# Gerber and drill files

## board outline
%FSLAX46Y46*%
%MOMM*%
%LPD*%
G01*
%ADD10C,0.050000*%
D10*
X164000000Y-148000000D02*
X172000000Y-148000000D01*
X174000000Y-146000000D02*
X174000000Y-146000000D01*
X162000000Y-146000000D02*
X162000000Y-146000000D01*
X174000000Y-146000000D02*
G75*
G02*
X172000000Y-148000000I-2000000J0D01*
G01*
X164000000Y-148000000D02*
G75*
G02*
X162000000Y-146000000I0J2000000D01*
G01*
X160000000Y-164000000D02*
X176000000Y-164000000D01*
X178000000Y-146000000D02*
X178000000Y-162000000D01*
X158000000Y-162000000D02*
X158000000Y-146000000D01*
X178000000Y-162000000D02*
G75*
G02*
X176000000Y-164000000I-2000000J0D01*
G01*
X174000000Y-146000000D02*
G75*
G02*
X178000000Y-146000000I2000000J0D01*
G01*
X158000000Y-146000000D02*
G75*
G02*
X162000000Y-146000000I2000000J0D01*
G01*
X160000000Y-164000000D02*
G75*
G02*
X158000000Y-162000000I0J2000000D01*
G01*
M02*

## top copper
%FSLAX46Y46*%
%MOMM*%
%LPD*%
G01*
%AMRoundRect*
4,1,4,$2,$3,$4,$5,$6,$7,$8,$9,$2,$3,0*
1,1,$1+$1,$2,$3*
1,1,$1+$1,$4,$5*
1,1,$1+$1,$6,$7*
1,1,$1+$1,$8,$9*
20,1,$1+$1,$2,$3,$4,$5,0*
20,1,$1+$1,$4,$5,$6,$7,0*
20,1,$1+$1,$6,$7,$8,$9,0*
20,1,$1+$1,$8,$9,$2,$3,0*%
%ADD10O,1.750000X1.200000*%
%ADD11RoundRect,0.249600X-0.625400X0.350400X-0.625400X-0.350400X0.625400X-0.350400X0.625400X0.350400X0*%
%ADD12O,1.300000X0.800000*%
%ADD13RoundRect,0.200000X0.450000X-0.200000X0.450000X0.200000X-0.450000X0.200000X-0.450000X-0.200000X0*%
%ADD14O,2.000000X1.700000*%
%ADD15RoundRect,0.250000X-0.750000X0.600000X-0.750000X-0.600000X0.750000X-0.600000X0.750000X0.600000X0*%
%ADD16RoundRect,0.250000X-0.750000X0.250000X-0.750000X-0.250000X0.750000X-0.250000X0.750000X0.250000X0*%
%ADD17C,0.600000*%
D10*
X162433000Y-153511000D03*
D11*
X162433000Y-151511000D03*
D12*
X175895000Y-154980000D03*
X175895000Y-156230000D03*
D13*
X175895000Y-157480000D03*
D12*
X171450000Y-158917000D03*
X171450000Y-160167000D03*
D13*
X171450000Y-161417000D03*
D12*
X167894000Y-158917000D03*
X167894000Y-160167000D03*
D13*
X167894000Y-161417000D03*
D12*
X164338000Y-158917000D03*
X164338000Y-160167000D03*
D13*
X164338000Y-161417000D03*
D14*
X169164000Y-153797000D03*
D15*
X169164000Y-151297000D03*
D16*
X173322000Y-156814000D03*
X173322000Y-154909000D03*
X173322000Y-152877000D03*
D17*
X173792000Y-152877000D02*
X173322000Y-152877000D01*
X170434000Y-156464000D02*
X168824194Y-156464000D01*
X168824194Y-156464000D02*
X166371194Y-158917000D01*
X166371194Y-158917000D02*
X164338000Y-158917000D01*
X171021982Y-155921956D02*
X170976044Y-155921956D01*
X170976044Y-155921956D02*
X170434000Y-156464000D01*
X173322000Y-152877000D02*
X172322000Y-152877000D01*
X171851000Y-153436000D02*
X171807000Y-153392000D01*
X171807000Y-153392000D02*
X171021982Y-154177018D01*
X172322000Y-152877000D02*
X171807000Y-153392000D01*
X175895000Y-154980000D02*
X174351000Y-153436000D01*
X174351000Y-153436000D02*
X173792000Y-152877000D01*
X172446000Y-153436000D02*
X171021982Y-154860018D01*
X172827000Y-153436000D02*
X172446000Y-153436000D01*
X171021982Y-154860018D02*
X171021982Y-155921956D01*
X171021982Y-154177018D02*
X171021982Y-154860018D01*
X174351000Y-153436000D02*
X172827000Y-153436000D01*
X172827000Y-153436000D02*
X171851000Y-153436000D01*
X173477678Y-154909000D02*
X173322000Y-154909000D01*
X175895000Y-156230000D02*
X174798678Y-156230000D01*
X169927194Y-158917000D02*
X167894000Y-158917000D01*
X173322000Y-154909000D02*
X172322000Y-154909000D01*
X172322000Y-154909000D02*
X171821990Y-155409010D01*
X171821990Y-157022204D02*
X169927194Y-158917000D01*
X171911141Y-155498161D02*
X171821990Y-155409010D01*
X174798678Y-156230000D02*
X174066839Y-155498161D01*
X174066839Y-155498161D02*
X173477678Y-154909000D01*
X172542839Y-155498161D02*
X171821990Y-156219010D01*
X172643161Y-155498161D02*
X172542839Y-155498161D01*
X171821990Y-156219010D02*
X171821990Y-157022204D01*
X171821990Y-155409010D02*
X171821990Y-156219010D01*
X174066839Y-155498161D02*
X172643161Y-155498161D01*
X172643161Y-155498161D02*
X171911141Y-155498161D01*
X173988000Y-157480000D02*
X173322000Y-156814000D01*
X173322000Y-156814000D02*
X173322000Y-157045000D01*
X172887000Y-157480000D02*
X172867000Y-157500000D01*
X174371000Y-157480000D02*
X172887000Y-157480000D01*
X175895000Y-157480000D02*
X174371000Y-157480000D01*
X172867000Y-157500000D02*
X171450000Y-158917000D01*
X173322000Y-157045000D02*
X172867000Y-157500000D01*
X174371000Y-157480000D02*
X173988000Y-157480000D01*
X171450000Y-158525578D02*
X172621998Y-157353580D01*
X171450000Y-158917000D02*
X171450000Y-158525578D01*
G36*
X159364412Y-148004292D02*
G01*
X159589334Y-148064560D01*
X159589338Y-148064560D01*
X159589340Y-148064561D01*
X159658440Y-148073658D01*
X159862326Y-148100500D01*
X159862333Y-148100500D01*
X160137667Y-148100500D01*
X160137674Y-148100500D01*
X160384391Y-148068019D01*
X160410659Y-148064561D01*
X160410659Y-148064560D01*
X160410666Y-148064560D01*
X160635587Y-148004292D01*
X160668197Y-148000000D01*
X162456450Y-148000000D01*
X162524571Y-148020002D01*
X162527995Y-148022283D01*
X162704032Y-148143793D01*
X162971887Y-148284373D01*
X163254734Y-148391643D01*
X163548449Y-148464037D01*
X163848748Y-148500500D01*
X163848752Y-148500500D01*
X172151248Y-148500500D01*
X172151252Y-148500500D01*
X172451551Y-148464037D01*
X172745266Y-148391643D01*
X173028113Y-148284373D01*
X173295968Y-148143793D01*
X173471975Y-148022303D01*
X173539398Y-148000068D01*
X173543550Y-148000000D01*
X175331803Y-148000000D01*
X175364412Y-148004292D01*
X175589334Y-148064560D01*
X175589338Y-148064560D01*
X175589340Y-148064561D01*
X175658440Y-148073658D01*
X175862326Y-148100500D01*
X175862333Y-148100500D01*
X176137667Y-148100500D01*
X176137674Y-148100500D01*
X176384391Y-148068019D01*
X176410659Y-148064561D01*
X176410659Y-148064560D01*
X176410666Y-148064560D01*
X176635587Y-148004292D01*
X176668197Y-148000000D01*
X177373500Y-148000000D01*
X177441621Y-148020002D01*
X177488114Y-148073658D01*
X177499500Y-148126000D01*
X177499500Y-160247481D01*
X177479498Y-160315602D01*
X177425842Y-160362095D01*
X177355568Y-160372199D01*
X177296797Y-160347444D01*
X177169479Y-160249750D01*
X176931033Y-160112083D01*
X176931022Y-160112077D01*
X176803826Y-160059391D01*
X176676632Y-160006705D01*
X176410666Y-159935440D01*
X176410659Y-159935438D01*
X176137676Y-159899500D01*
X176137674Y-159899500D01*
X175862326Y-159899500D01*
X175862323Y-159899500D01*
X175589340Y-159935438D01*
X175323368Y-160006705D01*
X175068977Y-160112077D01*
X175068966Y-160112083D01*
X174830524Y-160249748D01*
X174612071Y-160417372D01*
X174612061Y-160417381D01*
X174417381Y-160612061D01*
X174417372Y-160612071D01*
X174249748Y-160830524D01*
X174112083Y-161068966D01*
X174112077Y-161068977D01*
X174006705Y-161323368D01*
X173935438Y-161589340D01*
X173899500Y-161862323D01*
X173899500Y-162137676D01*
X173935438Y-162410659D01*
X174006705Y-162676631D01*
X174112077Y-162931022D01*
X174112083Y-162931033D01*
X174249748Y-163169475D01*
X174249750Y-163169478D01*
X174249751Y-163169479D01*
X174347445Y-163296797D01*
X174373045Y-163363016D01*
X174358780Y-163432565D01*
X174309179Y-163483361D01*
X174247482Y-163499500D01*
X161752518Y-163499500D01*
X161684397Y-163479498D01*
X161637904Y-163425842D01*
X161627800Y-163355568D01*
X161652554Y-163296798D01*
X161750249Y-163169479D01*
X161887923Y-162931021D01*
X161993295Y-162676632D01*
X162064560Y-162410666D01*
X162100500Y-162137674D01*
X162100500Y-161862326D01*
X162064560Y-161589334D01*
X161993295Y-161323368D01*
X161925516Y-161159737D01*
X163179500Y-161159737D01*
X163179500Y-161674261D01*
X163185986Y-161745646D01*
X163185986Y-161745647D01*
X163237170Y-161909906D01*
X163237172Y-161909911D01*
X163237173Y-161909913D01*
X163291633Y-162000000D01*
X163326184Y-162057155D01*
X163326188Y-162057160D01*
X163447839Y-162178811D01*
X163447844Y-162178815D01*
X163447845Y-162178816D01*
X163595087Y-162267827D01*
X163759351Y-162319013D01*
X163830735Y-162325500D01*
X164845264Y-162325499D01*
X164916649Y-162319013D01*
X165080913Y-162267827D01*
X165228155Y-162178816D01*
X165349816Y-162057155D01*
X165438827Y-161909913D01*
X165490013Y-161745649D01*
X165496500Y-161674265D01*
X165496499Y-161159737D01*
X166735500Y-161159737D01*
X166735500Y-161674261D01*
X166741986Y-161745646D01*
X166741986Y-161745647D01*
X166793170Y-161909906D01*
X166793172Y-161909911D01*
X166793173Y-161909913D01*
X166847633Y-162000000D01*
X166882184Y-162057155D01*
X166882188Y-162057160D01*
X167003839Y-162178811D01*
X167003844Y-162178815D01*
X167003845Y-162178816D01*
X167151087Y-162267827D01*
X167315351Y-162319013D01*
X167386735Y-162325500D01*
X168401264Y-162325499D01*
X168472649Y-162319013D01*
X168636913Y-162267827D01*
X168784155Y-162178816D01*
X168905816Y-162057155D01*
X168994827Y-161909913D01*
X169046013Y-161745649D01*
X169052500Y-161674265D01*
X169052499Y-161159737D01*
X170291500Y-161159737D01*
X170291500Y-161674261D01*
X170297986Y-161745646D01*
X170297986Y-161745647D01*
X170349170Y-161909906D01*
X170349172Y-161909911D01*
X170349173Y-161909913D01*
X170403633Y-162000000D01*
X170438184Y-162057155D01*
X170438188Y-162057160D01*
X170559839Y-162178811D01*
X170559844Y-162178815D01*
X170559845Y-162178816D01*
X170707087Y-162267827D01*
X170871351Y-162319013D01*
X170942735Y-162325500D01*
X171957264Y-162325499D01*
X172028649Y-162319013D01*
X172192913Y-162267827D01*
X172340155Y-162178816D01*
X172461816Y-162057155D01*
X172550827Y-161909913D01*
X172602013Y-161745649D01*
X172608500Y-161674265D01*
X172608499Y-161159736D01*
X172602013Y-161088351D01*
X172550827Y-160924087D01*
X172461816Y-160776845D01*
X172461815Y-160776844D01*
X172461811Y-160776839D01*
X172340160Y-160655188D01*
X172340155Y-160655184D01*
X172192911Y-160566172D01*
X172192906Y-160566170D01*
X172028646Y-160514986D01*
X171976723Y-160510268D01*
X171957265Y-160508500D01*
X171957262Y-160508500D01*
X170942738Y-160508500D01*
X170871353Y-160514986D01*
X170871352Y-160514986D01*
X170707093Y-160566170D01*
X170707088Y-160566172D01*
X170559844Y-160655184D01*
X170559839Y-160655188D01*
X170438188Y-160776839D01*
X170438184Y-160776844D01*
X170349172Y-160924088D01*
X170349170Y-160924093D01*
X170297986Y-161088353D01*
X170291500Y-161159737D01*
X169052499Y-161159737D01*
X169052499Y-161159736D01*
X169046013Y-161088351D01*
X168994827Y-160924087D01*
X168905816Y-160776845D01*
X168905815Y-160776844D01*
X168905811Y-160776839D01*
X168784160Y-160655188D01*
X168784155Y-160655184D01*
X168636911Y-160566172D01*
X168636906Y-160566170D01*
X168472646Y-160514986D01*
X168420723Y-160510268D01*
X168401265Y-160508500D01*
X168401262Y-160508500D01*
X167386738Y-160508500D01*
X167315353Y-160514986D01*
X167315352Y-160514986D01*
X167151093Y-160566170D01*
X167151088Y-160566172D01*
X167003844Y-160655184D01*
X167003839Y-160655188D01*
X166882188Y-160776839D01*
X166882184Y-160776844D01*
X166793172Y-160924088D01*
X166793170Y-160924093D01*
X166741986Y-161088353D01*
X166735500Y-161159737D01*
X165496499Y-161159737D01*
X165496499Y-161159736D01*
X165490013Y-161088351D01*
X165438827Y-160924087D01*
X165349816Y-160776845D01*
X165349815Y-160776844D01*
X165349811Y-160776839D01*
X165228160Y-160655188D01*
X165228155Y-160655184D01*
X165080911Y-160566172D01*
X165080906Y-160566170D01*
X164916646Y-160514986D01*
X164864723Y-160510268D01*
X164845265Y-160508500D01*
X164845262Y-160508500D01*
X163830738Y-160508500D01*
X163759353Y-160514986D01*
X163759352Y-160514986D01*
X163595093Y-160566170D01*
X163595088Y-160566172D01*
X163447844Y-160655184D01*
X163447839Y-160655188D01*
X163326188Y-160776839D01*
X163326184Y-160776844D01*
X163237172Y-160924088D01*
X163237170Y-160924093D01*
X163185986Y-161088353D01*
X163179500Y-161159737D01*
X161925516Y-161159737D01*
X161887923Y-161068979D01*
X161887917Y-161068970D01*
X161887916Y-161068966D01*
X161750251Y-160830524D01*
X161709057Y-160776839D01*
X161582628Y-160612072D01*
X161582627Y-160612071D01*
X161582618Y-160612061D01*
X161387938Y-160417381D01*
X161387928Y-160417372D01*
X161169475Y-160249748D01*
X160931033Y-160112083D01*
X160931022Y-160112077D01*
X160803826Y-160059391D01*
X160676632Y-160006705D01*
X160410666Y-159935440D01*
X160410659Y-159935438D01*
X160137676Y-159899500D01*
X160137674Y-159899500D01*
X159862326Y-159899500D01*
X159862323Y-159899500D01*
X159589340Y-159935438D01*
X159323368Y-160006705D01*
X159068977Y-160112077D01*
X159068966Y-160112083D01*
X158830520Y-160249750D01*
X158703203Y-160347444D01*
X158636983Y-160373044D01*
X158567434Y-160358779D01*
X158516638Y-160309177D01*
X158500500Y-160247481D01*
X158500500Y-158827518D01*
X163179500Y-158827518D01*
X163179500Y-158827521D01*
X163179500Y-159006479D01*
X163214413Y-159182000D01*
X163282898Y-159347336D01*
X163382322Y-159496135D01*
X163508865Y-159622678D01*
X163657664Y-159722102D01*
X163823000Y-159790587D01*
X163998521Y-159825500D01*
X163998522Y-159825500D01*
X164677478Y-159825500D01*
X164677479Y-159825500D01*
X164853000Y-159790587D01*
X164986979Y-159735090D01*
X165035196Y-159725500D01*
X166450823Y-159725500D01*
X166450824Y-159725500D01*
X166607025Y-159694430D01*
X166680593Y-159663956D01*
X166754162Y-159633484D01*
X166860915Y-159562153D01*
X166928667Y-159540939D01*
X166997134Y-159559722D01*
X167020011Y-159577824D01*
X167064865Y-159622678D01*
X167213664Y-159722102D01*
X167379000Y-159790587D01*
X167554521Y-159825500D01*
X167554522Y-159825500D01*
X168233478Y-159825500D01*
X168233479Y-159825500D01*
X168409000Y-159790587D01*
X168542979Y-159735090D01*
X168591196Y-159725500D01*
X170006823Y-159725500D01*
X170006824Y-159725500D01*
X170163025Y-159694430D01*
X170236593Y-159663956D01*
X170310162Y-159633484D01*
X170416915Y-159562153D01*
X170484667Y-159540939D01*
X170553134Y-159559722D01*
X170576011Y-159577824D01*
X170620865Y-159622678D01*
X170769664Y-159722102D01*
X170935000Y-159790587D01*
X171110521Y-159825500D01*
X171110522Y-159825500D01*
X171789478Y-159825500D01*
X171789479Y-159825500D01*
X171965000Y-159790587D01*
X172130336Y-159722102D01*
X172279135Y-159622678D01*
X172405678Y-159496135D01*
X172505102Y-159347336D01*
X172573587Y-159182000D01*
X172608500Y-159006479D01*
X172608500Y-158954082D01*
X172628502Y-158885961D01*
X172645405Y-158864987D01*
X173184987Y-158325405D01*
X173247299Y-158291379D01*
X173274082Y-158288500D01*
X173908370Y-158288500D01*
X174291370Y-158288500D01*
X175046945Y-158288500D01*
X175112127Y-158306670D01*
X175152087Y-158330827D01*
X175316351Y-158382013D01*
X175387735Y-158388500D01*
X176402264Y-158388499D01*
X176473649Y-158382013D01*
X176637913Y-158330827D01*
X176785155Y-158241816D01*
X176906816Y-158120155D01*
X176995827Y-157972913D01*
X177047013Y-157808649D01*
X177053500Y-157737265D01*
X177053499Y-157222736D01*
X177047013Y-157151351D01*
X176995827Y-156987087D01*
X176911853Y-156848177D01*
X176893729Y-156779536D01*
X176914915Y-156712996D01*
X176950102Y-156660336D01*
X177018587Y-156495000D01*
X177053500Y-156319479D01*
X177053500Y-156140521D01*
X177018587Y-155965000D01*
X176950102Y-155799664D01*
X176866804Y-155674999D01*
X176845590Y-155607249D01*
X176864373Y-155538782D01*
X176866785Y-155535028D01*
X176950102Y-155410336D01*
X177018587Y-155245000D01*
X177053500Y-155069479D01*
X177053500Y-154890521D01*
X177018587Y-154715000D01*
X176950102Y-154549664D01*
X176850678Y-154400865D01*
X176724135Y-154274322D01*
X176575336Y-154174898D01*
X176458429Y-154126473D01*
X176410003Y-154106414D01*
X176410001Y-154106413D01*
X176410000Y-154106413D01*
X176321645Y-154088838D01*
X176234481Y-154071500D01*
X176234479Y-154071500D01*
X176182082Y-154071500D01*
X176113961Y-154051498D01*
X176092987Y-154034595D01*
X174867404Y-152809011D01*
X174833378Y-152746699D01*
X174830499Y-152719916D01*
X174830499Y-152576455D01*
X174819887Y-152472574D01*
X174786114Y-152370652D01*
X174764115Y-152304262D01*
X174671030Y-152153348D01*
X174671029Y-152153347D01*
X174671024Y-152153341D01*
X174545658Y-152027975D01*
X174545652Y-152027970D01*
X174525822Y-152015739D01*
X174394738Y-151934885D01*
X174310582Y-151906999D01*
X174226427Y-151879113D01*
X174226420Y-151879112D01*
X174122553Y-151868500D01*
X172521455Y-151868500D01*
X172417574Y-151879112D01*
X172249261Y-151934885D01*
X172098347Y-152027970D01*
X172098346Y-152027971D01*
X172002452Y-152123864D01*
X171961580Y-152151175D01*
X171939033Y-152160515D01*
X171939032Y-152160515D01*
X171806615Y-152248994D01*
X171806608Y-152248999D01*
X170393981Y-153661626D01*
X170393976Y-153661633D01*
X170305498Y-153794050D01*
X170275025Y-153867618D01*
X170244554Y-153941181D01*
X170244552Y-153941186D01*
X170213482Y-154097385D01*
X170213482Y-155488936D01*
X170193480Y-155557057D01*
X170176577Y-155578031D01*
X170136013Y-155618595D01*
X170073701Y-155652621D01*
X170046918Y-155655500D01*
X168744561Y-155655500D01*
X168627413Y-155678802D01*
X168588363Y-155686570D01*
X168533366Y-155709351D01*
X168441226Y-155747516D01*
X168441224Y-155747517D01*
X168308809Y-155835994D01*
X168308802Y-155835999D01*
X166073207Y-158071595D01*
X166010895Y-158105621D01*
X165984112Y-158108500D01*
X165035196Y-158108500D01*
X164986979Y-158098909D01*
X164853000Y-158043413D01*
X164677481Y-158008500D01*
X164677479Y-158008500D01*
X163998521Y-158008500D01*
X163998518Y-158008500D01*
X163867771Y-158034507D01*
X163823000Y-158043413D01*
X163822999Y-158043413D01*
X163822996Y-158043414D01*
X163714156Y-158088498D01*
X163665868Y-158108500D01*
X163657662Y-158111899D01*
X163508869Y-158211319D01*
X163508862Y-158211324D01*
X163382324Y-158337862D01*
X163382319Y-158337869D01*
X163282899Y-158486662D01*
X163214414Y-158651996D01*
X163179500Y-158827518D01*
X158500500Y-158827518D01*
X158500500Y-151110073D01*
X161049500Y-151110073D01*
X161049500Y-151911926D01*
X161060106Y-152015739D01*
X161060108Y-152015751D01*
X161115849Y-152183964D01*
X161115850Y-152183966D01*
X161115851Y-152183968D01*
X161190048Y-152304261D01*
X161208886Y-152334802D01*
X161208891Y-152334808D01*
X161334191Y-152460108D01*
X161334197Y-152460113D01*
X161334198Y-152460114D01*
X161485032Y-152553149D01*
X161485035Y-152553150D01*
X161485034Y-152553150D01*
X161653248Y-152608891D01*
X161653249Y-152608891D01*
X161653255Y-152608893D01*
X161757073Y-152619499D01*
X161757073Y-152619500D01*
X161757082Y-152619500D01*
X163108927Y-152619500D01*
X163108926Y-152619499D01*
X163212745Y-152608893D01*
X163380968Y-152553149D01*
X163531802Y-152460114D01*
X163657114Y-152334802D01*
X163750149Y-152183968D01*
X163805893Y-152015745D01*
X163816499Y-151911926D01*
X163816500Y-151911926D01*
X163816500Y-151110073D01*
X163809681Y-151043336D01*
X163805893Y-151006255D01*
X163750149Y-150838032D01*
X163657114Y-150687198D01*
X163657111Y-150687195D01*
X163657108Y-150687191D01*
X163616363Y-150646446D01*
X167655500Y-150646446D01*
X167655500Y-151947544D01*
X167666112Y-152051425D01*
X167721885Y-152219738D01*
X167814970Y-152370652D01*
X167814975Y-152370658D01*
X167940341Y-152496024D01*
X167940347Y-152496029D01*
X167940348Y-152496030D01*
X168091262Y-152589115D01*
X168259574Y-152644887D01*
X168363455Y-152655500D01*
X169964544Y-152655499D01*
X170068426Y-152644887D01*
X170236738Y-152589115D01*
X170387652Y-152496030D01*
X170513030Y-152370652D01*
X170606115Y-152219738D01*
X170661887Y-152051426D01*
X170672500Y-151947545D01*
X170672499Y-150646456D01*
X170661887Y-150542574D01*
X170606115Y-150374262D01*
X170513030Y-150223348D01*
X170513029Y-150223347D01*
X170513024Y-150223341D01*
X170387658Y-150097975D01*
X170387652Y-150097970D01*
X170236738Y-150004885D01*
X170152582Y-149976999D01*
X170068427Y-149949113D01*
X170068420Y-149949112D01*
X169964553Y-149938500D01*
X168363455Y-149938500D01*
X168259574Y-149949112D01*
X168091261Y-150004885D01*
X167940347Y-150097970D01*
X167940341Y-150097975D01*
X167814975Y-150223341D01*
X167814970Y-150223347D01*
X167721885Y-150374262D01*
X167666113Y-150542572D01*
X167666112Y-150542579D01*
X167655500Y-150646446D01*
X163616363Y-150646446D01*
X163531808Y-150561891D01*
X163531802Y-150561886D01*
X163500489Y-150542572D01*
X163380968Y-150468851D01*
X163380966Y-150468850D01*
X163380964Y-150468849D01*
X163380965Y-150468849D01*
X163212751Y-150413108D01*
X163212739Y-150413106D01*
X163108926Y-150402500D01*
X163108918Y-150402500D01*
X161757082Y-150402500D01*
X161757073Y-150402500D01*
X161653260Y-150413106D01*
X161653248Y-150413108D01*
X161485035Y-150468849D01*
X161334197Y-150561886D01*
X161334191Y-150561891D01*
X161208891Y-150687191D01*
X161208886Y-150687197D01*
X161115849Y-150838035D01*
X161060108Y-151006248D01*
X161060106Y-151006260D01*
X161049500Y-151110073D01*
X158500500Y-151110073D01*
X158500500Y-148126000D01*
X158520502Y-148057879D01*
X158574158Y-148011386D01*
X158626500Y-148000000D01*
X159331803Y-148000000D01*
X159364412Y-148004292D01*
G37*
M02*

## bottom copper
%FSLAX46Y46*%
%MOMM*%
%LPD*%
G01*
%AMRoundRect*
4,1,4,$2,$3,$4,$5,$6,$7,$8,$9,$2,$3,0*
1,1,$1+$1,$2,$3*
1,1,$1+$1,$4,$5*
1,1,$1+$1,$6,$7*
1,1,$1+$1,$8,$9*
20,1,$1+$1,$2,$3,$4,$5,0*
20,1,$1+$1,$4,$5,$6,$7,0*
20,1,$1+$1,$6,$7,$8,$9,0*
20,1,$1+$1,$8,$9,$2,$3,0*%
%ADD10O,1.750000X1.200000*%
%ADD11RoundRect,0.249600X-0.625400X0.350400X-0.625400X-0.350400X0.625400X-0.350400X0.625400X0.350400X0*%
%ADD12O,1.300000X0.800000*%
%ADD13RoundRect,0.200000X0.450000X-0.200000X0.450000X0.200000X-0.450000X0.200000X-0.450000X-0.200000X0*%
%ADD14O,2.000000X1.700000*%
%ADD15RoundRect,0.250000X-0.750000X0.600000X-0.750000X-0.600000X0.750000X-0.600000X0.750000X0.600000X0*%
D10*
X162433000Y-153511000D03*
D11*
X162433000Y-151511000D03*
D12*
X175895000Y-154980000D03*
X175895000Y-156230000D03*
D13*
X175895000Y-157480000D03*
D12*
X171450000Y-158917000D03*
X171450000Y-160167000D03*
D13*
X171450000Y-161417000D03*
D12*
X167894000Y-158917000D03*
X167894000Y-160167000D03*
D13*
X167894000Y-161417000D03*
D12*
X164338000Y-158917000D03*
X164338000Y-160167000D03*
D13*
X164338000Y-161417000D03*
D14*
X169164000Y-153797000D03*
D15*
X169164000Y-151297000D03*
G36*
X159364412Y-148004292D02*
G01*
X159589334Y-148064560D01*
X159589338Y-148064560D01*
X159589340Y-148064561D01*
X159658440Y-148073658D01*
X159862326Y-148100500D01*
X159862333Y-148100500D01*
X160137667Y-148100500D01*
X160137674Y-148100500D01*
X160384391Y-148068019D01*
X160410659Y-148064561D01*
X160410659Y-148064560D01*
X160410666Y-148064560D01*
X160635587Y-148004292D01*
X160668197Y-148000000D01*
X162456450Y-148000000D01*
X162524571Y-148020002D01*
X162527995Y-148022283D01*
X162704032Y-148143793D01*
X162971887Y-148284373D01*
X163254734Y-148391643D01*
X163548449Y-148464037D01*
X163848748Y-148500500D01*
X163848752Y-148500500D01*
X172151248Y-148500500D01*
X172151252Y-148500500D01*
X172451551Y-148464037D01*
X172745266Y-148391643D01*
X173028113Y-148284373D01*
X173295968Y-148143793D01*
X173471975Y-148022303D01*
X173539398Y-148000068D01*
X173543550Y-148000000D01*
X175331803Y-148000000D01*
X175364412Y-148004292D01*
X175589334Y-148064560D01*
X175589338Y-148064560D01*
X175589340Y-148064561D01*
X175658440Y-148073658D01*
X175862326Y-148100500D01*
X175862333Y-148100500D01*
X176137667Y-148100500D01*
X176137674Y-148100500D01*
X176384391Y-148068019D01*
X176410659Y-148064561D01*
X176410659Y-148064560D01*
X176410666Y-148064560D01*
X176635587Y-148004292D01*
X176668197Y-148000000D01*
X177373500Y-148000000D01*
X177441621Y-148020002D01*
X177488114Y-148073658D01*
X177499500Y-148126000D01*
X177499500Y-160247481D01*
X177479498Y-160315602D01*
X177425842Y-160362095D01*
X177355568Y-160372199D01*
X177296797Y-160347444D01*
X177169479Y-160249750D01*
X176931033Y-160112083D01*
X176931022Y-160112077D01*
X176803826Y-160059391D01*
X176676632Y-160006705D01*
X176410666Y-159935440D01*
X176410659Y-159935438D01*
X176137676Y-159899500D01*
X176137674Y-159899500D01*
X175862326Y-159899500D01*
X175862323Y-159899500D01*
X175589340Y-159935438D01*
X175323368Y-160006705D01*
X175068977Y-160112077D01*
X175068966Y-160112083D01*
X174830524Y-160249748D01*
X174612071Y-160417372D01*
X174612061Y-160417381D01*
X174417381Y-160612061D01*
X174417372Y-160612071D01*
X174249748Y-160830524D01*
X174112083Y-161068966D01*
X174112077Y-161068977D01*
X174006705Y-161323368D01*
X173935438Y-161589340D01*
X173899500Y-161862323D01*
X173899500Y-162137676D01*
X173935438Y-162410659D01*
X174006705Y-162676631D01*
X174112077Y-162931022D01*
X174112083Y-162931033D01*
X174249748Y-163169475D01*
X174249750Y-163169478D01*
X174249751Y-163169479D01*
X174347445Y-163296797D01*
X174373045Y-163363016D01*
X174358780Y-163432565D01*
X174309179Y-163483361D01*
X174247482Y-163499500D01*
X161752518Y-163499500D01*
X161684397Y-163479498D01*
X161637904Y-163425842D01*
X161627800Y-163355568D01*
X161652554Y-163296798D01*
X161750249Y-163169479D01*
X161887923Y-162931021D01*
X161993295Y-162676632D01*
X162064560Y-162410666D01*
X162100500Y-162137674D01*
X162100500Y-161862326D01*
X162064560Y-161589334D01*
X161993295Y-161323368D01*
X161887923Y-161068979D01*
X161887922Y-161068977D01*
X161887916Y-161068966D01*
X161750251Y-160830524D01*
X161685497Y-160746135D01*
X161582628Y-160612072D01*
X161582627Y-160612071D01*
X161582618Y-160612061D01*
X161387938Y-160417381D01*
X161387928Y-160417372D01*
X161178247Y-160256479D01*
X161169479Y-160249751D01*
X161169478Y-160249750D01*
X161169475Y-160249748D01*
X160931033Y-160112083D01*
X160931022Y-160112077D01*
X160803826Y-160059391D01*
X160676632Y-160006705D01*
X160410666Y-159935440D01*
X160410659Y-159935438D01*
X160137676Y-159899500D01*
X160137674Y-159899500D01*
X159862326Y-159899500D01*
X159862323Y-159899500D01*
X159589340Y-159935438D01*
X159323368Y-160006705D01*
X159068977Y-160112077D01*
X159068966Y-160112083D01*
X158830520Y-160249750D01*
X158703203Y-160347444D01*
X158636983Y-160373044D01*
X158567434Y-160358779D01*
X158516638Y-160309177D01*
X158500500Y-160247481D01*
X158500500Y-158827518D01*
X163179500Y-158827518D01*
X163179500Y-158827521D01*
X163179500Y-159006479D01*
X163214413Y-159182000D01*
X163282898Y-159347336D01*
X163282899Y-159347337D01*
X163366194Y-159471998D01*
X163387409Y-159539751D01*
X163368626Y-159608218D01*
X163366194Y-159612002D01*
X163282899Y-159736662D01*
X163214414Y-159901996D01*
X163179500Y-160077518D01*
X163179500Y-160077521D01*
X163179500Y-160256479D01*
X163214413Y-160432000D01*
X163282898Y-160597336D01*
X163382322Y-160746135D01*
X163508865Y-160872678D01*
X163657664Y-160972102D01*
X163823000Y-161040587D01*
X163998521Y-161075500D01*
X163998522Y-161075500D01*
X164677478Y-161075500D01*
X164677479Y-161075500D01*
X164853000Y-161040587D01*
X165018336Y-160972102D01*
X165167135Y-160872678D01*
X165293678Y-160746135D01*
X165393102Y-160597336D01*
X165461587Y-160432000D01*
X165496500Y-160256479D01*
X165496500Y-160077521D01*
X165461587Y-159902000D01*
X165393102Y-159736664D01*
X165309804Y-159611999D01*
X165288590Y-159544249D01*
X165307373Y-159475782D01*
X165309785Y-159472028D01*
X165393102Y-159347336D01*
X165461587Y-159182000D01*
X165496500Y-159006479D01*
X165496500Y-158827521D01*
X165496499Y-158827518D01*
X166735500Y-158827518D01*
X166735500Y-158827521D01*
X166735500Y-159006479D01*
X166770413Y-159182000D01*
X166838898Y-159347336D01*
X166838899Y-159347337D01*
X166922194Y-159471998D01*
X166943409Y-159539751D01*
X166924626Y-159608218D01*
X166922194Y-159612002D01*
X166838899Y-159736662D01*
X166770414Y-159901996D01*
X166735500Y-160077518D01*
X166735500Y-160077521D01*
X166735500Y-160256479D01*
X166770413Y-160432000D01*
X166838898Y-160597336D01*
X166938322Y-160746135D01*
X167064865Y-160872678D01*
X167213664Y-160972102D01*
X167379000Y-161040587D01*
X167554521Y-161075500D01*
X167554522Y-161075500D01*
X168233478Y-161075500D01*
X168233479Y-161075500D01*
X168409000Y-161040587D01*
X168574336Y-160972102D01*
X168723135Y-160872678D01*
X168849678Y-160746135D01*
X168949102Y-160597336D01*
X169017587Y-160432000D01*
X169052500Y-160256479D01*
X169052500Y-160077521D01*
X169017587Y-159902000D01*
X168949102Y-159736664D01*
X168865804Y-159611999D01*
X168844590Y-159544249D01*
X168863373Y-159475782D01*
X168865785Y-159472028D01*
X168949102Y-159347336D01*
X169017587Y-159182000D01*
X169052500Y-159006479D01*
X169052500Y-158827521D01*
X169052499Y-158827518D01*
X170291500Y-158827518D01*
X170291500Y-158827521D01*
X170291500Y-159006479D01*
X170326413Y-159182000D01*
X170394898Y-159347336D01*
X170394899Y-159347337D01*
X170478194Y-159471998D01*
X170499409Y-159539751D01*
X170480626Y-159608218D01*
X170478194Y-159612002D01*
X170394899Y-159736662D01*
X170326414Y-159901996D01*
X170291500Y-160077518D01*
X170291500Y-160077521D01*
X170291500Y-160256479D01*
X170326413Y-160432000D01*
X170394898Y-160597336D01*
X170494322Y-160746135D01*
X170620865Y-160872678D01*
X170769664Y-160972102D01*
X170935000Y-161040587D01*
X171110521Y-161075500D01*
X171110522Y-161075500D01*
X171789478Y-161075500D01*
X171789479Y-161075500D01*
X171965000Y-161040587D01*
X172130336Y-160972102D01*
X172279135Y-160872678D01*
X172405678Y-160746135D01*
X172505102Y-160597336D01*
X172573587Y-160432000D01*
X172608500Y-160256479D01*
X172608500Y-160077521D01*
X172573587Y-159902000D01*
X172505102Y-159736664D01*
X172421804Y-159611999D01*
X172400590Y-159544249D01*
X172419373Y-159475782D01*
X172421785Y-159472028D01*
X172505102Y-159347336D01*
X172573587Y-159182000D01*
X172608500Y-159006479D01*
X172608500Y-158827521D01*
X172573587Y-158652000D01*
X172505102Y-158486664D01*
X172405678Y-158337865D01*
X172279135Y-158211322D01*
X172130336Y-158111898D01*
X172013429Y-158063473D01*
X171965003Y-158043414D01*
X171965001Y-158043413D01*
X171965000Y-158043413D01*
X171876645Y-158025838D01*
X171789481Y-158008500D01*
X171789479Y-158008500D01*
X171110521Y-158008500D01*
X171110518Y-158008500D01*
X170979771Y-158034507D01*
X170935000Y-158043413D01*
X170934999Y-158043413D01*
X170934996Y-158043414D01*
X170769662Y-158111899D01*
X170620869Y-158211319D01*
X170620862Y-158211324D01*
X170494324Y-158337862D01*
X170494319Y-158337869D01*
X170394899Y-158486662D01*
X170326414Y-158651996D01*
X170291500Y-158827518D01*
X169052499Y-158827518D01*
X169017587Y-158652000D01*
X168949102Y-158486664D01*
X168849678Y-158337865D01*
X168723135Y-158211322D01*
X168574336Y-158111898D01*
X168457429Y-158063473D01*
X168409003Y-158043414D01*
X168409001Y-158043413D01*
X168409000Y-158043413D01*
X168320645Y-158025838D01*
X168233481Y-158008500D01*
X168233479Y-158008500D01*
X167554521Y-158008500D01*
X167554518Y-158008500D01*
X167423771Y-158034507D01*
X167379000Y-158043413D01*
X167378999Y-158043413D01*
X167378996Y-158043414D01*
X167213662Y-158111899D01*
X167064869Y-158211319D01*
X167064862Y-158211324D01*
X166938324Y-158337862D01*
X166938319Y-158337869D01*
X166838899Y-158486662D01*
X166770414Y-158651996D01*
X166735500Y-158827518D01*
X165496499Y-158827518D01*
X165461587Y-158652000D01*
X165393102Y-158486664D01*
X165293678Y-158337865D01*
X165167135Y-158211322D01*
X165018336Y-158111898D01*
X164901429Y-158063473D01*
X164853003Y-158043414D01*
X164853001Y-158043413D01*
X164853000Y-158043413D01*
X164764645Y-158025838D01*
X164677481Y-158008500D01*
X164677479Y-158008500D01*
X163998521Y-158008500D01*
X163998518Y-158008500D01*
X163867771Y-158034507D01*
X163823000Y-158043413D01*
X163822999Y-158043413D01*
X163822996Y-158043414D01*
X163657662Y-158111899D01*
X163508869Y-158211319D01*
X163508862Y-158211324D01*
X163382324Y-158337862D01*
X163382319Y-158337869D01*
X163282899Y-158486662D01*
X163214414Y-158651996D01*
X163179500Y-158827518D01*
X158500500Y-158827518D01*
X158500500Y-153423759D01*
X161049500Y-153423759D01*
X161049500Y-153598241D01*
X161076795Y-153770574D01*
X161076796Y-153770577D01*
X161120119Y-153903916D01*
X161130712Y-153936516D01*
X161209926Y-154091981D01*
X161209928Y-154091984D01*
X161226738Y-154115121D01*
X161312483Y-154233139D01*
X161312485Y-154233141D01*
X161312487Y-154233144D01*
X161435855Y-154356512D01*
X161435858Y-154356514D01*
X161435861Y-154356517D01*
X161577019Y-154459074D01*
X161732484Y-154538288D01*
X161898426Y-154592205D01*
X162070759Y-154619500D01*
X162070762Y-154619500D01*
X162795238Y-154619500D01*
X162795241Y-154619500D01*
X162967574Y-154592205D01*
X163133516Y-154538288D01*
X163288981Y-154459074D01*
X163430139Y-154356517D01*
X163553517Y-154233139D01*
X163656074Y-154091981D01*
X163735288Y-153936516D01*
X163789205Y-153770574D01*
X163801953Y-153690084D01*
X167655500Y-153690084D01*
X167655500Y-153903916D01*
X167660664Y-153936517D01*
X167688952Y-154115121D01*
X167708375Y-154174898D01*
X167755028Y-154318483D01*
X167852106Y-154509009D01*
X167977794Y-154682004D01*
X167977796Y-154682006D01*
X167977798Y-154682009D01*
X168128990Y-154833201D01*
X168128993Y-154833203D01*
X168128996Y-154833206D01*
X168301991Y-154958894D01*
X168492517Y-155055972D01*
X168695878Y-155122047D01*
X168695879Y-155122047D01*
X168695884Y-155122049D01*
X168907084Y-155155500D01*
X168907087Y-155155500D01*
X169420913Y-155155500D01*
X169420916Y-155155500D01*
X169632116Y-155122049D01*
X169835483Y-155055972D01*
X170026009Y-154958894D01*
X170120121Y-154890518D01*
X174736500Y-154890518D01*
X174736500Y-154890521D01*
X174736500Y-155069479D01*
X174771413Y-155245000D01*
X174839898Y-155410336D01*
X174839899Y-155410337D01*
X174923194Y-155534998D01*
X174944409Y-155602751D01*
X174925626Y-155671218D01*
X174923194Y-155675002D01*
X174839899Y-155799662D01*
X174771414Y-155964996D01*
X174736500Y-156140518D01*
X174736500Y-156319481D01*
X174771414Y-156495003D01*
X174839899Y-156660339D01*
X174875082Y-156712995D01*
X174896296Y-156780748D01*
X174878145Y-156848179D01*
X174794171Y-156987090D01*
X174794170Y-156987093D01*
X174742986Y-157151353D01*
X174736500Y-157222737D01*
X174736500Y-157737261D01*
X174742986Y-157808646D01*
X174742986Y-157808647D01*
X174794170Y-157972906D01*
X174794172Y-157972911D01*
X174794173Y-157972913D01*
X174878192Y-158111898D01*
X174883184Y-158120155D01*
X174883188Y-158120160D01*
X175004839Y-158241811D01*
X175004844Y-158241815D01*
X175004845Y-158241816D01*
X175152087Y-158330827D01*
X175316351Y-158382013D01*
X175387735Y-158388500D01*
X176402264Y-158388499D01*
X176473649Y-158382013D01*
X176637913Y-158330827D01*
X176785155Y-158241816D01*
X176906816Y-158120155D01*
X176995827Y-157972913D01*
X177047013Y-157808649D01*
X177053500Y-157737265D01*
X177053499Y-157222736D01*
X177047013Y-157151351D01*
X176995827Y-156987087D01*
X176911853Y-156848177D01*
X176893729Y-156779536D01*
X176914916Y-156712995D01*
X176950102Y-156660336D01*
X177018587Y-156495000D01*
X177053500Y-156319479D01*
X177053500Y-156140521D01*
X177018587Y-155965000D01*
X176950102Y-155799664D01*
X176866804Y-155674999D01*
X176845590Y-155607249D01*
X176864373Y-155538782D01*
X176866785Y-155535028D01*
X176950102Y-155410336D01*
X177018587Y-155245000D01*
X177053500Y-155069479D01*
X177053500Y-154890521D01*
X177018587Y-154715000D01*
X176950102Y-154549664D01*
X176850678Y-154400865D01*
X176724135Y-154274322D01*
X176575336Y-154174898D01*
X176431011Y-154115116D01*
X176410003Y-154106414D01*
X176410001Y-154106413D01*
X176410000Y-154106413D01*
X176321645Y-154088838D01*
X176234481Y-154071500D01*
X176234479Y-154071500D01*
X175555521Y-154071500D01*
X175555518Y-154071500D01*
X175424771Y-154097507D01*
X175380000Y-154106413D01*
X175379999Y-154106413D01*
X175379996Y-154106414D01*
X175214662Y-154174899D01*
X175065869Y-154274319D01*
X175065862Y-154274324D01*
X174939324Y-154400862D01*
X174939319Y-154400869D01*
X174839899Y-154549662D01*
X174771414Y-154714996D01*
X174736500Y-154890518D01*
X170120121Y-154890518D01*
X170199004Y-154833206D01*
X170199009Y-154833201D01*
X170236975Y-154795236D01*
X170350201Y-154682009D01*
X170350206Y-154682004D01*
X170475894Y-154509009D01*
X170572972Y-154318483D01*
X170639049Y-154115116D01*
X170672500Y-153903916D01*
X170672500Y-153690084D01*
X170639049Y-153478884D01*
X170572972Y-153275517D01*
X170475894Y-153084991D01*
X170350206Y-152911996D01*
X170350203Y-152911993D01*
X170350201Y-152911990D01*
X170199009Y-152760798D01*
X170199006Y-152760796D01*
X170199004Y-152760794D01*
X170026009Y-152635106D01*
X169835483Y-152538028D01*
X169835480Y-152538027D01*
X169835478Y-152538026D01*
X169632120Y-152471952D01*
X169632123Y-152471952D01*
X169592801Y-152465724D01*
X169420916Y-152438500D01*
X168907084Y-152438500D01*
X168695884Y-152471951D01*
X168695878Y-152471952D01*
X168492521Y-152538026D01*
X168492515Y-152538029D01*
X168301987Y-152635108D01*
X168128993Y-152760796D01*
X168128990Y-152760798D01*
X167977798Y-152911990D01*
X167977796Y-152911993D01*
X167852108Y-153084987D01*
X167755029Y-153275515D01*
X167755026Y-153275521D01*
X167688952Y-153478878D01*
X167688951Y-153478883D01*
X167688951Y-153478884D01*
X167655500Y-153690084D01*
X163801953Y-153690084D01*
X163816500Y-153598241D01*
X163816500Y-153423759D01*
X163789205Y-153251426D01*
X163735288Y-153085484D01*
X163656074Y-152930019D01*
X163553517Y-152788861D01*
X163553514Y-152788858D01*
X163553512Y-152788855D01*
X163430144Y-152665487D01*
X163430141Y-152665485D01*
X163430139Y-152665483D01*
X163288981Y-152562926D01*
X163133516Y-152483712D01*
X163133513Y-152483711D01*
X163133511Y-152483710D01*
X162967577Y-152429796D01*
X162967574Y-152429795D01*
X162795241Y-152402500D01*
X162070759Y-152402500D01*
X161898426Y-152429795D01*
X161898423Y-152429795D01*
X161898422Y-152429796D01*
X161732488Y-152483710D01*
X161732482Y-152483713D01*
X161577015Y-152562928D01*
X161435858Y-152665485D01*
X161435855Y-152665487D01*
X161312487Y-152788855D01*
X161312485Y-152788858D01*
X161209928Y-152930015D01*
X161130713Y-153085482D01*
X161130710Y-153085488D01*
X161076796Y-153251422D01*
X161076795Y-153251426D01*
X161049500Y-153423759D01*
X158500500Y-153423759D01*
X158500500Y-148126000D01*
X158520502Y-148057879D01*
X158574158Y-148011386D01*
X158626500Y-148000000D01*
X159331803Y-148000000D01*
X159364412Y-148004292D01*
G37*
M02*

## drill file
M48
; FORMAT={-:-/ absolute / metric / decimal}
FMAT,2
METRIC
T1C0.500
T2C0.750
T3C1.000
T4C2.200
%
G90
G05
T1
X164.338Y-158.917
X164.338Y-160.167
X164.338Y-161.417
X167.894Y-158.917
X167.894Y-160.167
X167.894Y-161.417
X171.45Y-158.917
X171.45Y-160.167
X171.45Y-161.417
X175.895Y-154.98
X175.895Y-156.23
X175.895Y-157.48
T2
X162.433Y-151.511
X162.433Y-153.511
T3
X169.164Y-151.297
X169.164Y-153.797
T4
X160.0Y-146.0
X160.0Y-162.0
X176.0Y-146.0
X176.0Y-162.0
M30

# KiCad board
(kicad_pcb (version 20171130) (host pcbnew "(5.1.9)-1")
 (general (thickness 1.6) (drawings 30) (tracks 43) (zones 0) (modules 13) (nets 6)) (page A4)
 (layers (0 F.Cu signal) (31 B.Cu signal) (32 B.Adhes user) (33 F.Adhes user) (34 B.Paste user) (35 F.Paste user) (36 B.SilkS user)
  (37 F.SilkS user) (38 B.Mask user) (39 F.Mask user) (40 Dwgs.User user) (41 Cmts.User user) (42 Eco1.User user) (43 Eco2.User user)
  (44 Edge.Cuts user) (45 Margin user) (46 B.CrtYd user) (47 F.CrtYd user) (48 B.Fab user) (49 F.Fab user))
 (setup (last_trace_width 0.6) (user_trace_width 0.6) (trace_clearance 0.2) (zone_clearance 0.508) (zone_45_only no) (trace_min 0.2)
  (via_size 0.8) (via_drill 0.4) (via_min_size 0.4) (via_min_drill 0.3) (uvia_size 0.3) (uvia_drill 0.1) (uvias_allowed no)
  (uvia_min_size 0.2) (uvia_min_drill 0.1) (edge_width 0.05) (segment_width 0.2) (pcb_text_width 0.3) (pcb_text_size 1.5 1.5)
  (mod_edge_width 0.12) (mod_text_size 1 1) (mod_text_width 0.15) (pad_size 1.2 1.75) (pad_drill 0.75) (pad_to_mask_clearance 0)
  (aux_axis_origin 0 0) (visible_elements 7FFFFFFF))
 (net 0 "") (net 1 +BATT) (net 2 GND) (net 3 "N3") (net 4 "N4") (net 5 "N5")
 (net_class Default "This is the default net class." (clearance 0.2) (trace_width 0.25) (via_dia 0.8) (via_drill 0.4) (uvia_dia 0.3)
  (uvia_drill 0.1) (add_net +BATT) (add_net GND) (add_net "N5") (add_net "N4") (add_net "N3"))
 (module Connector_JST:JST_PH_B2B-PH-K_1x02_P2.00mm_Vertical (layer B.Cu) (at 162.433 151.511 270)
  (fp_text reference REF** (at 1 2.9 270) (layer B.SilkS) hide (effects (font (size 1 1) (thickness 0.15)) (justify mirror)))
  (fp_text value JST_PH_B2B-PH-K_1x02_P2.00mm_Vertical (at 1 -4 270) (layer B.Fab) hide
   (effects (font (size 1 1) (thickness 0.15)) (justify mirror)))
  (pad 2 thru_hole oval (at 2 0 270) (size 1.2 1.75) (drill 0.75) (layers *.Cu *.Mask) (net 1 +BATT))
  (pad 1 thru_hole roundrect (at 0 0 270) (size 1.2 1.75) (drill 0.75) (layers *.Cu *.Mask) (roundrect_rratio 0.208) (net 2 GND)))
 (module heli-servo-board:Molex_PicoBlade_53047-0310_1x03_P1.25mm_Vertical (layer F.Cu) (at 175.895 157.48 90)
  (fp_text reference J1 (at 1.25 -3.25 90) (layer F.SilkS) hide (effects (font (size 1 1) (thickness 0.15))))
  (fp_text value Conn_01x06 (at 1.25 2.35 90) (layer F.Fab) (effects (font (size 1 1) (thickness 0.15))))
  (pad 3 thru_hole oval (at 2.5 0 90) (size 0.8 1.3) (drill 0.5) (layers *.Cu *.Mask) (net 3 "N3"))
  (pad 2 thru_hole oval (at 1.25 0 90) (size 0.8 1.3) (drill 0.5) (layers *.Cu *.Mask) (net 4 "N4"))
  (pad 1 thru_hole roundrect (at 0 0 90) (size 0.8 1.3) (drill 0.5) (layers *.Cu *.Mask) (roundrect_rratio 0.25) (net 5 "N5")))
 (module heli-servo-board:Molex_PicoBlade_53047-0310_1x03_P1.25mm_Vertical (layer F.Cu) (at 171.45 161.417 90)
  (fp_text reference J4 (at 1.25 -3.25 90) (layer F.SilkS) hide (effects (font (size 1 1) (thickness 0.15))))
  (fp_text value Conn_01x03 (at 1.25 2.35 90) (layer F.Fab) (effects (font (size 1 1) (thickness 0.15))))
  (pad 3 thru_hole oval (at 2.5 0 90) (size 0.8 1.3) (drill 0.5) (layers *.Cu *.Mask) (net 5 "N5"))
  (pad 2 thru_hole oval (at 1.25 0 90) (size 0.8 1.3) (drill 0.5) (layers *.Cu *.Mask) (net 1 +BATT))
  (pad 1 thru_hole roundrect (at 0 0 90) (size 0.8 1.3) (drill 0.5) (layers *.Cu *.Mask) (roundrect_rratio 0.25) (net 2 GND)))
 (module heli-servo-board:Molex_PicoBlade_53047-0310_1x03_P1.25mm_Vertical (layer F.Cu) (at 167.894 161.417 90)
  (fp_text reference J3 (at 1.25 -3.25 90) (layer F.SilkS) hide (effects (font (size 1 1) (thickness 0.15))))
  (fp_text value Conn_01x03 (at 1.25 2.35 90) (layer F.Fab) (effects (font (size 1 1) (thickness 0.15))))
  (pad 3 thru_hole oval (at 2.5 0 90) (size 0.8 1.3) (drill 0.5) (layers *.Cu *.Mask) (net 4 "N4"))
  (pad 2 thru_hole oval (at 1.25 0 90) (size 0.8 1.3) (drill 0.5) (layers *.Cu *.Mask) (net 1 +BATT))
  (pad 1 thru_hole roundrect (at 0 0 90) (size 0.8 1.3) (drill 0.5) (layers *.Cu *.Mask) (roundrect_rratio 0.25) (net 2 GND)))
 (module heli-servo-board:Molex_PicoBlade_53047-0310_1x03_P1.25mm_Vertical (layer F.Cu) (at 164.338 161.417 90)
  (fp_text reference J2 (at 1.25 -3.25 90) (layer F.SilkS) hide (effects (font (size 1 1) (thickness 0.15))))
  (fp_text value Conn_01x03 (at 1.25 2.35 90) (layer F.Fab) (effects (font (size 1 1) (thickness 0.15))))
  (pad 3 thru_hole oval (at 2.5 0 90) (size 0.8 1.3) (drill 0.5) (layers *.Cu *.Mask) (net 3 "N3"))
  (pad 2 thru_hole oval (at 1.25 0 90) (size 0.8 1.3) (drill 0.5) (layers *.Cu *.Mask) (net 1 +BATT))
  (pad 1 thru_hole roundrect (at 0 0 90) (size 0.8 1.3) (drill 0.5) (layers *.Cu *.Mask) (roundrect_rratio 0.25) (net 2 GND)))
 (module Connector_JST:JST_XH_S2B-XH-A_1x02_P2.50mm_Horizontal (layer F.Cu) (at 169.164 151.297 270)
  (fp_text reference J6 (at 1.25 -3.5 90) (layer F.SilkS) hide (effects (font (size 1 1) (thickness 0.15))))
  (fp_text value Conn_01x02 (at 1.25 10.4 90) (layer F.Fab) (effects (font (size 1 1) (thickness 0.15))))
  (pad 2 thru_hole oval (at 2.5 0 270) (size 1.7 2) (drill 1) (layers *.Cu *.Mask) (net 1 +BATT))
  (pad 1 thru_hole roundrect (at 0 0 270) (size 1.7 2) (drill 1) (layers *.Cu *.Mask) (roundrect_rratio 0.1470588235294118) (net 2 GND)))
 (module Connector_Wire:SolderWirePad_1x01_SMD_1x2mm (layer F.Cu) (at 173.322 156.814 270)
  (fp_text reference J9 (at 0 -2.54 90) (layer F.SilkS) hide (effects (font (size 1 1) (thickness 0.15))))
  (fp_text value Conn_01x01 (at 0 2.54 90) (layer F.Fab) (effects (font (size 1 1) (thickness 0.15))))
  (pad 1 smd roundrect (at 0 0 270) (size 1 2) (layers F.Cu F.Paste F.Mask) (roundrect_rratio 0.25) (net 5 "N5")))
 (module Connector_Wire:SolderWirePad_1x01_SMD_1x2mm (layer F.Cu) (at 173.322 154.909 270)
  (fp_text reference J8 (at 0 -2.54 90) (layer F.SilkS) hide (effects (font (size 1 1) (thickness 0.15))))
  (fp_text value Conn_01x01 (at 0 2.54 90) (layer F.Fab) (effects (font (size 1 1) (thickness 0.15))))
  (pad 1 smd roundrect (at 0 0 270) (size 1 2) (layers F.Cu F.Paste F.Mask) (roundrect_rratio 0.25) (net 4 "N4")))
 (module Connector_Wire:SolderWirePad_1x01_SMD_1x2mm (layer F.Cu) (at 173.322 152.877 270)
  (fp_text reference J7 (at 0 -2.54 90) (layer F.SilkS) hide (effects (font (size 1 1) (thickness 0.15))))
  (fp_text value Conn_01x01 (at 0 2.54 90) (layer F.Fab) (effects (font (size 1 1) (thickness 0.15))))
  (pad 1 smd roundrect (at 0 0 270) (size 1 2) (layers F.Cu F.Paste F.Mask) (roundrect_rratio 0.25) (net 3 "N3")))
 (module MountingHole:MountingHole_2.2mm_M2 (layer F.Cu) (at 176 162)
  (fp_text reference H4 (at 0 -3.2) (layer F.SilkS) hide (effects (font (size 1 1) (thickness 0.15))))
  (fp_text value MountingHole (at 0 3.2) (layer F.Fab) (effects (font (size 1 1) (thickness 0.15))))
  (pad "" np_thru_hole circle (at 0 0) (size 2.2 2.2) (drill 2.2) (layers *.Cu *.Mask) (clearance 1)))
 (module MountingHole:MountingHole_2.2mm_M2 (layer F.Cu) (at 176 146)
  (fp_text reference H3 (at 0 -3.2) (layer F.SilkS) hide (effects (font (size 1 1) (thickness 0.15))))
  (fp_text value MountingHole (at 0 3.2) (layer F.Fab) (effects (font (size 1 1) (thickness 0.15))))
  (pad "" np_thru_hole circle (at 0 0) (size 2.2 2.2) (drill 2.2) (layers *.Cu *.Mask) (clearance 1)))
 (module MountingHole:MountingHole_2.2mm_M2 (layer F.Cu) (at 160 162)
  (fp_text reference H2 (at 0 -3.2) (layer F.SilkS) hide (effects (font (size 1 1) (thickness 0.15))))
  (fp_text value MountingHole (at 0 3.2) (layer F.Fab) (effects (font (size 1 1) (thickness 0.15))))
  (pad "" np_thru_hole circle (at 0 0) (size 2.2 2.2) (drill 2.2) (layers *.Cu *.Mask) (clearance 1)))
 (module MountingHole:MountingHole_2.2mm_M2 (layer F.Cu) (at 160 146)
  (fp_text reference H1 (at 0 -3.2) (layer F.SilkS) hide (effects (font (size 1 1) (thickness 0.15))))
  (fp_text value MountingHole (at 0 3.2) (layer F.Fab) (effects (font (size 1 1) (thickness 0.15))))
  (pad "" np_thru_hole circle (at 0 0) (size 2.2 2.2) (drill 2.2) (layers *.Cu *.Mask) (clearance 1)))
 (gr_line (start 164 148) (end 172 148) (layer Edge.Cuts) (width 0.05))
 (gr_line (start 174 146) (end 174 146) (layer Edge.Cuts) (width 0.05))
 (gr_line (start 162 146) (end 162 146) (layer Edge.Cuts) (width 0.05))
 (gr_arc (start 172 146) (end 172 148) (angle -90) (layer Edge.Cuts) (width 0.05))
 (gr_arc (start 164 146) (end 162 146) (angle -90) (layer Edge.Cuts) (width 0.05))
 (gr_line (start 160 164) (end 176 164) (layer Edge.Cuts) (width 0.05))
 (gr_line (start 178 146) (end 178 162) (layer Edge.Cuts) (width 0.05))
 (gr_line (start 158 162) (end 158 146) (layer Edge.Cuts) (width 0.05))
 (gr_arc (start 176 162) (end 176 164) (angle -90) (layer Edge.Cuts) (width 0.05))
 (gr_arc (start 176 146) (end 178 146) (angle -180) (layer Edge.Cuts) (width 0.05))
 (gr_arc (start 160 146) (end 162 146) (angle -180) (layer Edge.Cuts) (width 0.05))
 (gr_arc (start 160 162) (end 158 162) (angle -90) (layer Edge.Cuts) (width 0.05))
 (segment (start 173.792 152.877) (end 173.322 152.877) (width 0.6) (layer F.Cu) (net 3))
 (segment (start 170.434 156.464) (end 168.824194 156.464) (width 0.6) (layer F.Cu) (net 3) (status 1000000))
 (segment (start 168.824194 156.464) (end 166.371194 158.917) (width 0.6) (layer F.Cu) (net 3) (status 1000000))
 (segment (start 166.371194 158.917) (end 164.338 158.917) (width 0.6) (layer F.Cu) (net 3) (status 1000000))
 (segment (start 171.021982 155.921956) (end 170.976044 155.921956) (width 0.6) (layer F.Cu) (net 3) (status 1000000))
 (segment (start 170.976044 155.921956) (end 170.434 156.464) (width 0.6) (layer F.Cu) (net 3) (status 1000000))
 (segment (start 173.322 152.877) (end 172.322 152.877) (width 0.6) (layer F.Cu) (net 3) (status 1000000))
 (segment (start 171.851 153.436) (end 171.807 153.392) (width 0.6) (layer F.Cu) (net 3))
 (segment (start 171.807 153.392) (end 171.021982 154.177018) (width 0.6) (layer F.Cu) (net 3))
 (segment (start 172.322 152.877) (end 171.807 153.392) (width 0.6) (layer F.Cu) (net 3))
 (segment (start 175.895 154.98) (end 174.351 153.436) (width 0.6) (layer F.Cu) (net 3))
 (segment (start 174.351 153.436) (end 173.792 152.877) (width 0.6) (layer F.Cu) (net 3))
 (segment (start 172.446 153.436) (end 171.021982 154.860018) (width 0.6) (layer F.Cu) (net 3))
 (segment (start 172.827 153.436) (end 172.446 153.436) (width 0.6) (layer F.Cu) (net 3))
 (segment (start 171.021982 154.860018) (end 171.021982 155.921956) (width 0.6) (layer F.Cu) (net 3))
 (segment (start 171.021982 154.177018) (end 171.021982 154.860018) (width 0.6) (layer F.Cu) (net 3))
 (segment (start 174.351 153.436) (end 172.827 153.436) (width 0.6) (layer F.Cu) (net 3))
 (segment (start 172.827 153.436) (end 171.851 153.436) (width 0.6) (layer F.Cu) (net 3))
 (segment (start 173.477678 154.909) (end 173.322 154.909) (width 0.6) (layer F.Cu) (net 4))
 (segment (start 175.895 156.23) (end 174.798678 156.23) (width 0.6) (layer F.Cu) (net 4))
 (segment (start 169.927194 158.917) (end 167.894 158.917) (width 0.6) (layer F.Cu) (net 4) (status 1000000))
 (segment (start 173.322 154.909) (end 172.322 154.909) (width 0.6) (layer F.Cu) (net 4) (status 1000000))
 (segment (start 172.322 154.909) (end 171.82199 155.40901) (width 0.6) (layer F.Cu) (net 4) (status 1000000))
 (segment (start 171.82199 157.022204) (end 169.927194 158.917) (width 0.6) (layer F.Cu) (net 4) (status 1000000))
 (segment (start 171.911141 155.498161) (end 171.82199 155.40901) (width 0.6) (layer F.Cu) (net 4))
 (segment (start 174.798678 156.23) (end 174.066839 155.498161) (width 0.6) (layer F.Cu) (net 4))
 (segment (start 174.066839 155.498161) (end 173.477678 154.909) (width 0.6) (layer F.Cu) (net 4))
 (segment (start 172.542839 155.498161) (end 171.82199 156.21901) (width 0.6) (layer F.Cu) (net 4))
 (segment (start 172.643161 155.498161) (end 172.542839 155.498161) (width 0.6) (layer F.Cu) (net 4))
 (segment (start 171.82199 156.21901) (end 171.82199 157.022204) (width 0.6) (layer F.Cu) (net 4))
 (segment (start 171.82199 155.40901) (end 171.82199 156.21901) (width 0.6) (layer F.Cu) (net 4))
 (segment (start 174.066839 155.498161) (end 172.643161 155.498161) (width 0.6) (layer F.Cu) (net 4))
 (segment (start 172.643161 155.498161) (end 171.911141 155.498161) (width 0.6) (layer F.Cu) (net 4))
 (segment (start 173.988 157.48) (end 173.322 156.814) (width 0.6) (layer F.Cu) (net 5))
 (segment (start 173.322 156.814) (end 173.322 157.045) (width 0.6) (layer F.Cu) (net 5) (status 1000000))
 (segment (start 172.887 157.48) (end 172.867 157.5) (width 0.6) (layer F.Cu) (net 5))
 (segment (start 174.371 157.48) (end 172.887 157.48) (width 0.6) (layer F.Cu) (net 5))
 (segment (start 175.895 157.48) (end 174.371 157.48) (width 0.6) (layer F.Cu) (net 5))
 (segment (start 172.867 157.5) (end 171.45 158.917) (width 0.6) (layer F.Cu) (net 5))
 (segment (start 173.322 157.045) (end 172.867 157.5) (width 0.6) (layer F.Cu) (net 5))
 (segment (start 174.371 157.48) (end 173.988 157.48) (width 0.6) (layer F.Cu) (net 5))
 (segment (start 171.45 158.525578) (end 172.621998 157.35358) (width 0.6) (layer F.Cu) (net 5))
 (segment (start 171.45 158.917) (end 171.45 158.525578) (width 0.6) (layer F.Cu) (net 5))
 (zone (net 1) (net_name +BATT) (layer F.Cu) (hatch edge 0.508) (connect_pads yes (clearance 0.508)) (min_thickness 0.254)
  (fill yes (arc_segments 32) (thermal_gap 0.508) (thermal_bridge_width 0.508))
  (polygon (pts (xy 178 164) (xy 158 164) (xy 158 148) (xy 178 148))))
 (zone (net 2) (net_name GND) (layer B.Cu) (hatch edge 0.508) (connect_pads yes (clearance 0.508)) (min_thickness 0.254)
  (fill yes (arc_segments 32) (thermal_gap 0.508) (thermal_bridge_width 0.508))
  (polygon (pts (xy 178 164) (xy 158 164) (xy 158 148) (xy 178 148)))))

